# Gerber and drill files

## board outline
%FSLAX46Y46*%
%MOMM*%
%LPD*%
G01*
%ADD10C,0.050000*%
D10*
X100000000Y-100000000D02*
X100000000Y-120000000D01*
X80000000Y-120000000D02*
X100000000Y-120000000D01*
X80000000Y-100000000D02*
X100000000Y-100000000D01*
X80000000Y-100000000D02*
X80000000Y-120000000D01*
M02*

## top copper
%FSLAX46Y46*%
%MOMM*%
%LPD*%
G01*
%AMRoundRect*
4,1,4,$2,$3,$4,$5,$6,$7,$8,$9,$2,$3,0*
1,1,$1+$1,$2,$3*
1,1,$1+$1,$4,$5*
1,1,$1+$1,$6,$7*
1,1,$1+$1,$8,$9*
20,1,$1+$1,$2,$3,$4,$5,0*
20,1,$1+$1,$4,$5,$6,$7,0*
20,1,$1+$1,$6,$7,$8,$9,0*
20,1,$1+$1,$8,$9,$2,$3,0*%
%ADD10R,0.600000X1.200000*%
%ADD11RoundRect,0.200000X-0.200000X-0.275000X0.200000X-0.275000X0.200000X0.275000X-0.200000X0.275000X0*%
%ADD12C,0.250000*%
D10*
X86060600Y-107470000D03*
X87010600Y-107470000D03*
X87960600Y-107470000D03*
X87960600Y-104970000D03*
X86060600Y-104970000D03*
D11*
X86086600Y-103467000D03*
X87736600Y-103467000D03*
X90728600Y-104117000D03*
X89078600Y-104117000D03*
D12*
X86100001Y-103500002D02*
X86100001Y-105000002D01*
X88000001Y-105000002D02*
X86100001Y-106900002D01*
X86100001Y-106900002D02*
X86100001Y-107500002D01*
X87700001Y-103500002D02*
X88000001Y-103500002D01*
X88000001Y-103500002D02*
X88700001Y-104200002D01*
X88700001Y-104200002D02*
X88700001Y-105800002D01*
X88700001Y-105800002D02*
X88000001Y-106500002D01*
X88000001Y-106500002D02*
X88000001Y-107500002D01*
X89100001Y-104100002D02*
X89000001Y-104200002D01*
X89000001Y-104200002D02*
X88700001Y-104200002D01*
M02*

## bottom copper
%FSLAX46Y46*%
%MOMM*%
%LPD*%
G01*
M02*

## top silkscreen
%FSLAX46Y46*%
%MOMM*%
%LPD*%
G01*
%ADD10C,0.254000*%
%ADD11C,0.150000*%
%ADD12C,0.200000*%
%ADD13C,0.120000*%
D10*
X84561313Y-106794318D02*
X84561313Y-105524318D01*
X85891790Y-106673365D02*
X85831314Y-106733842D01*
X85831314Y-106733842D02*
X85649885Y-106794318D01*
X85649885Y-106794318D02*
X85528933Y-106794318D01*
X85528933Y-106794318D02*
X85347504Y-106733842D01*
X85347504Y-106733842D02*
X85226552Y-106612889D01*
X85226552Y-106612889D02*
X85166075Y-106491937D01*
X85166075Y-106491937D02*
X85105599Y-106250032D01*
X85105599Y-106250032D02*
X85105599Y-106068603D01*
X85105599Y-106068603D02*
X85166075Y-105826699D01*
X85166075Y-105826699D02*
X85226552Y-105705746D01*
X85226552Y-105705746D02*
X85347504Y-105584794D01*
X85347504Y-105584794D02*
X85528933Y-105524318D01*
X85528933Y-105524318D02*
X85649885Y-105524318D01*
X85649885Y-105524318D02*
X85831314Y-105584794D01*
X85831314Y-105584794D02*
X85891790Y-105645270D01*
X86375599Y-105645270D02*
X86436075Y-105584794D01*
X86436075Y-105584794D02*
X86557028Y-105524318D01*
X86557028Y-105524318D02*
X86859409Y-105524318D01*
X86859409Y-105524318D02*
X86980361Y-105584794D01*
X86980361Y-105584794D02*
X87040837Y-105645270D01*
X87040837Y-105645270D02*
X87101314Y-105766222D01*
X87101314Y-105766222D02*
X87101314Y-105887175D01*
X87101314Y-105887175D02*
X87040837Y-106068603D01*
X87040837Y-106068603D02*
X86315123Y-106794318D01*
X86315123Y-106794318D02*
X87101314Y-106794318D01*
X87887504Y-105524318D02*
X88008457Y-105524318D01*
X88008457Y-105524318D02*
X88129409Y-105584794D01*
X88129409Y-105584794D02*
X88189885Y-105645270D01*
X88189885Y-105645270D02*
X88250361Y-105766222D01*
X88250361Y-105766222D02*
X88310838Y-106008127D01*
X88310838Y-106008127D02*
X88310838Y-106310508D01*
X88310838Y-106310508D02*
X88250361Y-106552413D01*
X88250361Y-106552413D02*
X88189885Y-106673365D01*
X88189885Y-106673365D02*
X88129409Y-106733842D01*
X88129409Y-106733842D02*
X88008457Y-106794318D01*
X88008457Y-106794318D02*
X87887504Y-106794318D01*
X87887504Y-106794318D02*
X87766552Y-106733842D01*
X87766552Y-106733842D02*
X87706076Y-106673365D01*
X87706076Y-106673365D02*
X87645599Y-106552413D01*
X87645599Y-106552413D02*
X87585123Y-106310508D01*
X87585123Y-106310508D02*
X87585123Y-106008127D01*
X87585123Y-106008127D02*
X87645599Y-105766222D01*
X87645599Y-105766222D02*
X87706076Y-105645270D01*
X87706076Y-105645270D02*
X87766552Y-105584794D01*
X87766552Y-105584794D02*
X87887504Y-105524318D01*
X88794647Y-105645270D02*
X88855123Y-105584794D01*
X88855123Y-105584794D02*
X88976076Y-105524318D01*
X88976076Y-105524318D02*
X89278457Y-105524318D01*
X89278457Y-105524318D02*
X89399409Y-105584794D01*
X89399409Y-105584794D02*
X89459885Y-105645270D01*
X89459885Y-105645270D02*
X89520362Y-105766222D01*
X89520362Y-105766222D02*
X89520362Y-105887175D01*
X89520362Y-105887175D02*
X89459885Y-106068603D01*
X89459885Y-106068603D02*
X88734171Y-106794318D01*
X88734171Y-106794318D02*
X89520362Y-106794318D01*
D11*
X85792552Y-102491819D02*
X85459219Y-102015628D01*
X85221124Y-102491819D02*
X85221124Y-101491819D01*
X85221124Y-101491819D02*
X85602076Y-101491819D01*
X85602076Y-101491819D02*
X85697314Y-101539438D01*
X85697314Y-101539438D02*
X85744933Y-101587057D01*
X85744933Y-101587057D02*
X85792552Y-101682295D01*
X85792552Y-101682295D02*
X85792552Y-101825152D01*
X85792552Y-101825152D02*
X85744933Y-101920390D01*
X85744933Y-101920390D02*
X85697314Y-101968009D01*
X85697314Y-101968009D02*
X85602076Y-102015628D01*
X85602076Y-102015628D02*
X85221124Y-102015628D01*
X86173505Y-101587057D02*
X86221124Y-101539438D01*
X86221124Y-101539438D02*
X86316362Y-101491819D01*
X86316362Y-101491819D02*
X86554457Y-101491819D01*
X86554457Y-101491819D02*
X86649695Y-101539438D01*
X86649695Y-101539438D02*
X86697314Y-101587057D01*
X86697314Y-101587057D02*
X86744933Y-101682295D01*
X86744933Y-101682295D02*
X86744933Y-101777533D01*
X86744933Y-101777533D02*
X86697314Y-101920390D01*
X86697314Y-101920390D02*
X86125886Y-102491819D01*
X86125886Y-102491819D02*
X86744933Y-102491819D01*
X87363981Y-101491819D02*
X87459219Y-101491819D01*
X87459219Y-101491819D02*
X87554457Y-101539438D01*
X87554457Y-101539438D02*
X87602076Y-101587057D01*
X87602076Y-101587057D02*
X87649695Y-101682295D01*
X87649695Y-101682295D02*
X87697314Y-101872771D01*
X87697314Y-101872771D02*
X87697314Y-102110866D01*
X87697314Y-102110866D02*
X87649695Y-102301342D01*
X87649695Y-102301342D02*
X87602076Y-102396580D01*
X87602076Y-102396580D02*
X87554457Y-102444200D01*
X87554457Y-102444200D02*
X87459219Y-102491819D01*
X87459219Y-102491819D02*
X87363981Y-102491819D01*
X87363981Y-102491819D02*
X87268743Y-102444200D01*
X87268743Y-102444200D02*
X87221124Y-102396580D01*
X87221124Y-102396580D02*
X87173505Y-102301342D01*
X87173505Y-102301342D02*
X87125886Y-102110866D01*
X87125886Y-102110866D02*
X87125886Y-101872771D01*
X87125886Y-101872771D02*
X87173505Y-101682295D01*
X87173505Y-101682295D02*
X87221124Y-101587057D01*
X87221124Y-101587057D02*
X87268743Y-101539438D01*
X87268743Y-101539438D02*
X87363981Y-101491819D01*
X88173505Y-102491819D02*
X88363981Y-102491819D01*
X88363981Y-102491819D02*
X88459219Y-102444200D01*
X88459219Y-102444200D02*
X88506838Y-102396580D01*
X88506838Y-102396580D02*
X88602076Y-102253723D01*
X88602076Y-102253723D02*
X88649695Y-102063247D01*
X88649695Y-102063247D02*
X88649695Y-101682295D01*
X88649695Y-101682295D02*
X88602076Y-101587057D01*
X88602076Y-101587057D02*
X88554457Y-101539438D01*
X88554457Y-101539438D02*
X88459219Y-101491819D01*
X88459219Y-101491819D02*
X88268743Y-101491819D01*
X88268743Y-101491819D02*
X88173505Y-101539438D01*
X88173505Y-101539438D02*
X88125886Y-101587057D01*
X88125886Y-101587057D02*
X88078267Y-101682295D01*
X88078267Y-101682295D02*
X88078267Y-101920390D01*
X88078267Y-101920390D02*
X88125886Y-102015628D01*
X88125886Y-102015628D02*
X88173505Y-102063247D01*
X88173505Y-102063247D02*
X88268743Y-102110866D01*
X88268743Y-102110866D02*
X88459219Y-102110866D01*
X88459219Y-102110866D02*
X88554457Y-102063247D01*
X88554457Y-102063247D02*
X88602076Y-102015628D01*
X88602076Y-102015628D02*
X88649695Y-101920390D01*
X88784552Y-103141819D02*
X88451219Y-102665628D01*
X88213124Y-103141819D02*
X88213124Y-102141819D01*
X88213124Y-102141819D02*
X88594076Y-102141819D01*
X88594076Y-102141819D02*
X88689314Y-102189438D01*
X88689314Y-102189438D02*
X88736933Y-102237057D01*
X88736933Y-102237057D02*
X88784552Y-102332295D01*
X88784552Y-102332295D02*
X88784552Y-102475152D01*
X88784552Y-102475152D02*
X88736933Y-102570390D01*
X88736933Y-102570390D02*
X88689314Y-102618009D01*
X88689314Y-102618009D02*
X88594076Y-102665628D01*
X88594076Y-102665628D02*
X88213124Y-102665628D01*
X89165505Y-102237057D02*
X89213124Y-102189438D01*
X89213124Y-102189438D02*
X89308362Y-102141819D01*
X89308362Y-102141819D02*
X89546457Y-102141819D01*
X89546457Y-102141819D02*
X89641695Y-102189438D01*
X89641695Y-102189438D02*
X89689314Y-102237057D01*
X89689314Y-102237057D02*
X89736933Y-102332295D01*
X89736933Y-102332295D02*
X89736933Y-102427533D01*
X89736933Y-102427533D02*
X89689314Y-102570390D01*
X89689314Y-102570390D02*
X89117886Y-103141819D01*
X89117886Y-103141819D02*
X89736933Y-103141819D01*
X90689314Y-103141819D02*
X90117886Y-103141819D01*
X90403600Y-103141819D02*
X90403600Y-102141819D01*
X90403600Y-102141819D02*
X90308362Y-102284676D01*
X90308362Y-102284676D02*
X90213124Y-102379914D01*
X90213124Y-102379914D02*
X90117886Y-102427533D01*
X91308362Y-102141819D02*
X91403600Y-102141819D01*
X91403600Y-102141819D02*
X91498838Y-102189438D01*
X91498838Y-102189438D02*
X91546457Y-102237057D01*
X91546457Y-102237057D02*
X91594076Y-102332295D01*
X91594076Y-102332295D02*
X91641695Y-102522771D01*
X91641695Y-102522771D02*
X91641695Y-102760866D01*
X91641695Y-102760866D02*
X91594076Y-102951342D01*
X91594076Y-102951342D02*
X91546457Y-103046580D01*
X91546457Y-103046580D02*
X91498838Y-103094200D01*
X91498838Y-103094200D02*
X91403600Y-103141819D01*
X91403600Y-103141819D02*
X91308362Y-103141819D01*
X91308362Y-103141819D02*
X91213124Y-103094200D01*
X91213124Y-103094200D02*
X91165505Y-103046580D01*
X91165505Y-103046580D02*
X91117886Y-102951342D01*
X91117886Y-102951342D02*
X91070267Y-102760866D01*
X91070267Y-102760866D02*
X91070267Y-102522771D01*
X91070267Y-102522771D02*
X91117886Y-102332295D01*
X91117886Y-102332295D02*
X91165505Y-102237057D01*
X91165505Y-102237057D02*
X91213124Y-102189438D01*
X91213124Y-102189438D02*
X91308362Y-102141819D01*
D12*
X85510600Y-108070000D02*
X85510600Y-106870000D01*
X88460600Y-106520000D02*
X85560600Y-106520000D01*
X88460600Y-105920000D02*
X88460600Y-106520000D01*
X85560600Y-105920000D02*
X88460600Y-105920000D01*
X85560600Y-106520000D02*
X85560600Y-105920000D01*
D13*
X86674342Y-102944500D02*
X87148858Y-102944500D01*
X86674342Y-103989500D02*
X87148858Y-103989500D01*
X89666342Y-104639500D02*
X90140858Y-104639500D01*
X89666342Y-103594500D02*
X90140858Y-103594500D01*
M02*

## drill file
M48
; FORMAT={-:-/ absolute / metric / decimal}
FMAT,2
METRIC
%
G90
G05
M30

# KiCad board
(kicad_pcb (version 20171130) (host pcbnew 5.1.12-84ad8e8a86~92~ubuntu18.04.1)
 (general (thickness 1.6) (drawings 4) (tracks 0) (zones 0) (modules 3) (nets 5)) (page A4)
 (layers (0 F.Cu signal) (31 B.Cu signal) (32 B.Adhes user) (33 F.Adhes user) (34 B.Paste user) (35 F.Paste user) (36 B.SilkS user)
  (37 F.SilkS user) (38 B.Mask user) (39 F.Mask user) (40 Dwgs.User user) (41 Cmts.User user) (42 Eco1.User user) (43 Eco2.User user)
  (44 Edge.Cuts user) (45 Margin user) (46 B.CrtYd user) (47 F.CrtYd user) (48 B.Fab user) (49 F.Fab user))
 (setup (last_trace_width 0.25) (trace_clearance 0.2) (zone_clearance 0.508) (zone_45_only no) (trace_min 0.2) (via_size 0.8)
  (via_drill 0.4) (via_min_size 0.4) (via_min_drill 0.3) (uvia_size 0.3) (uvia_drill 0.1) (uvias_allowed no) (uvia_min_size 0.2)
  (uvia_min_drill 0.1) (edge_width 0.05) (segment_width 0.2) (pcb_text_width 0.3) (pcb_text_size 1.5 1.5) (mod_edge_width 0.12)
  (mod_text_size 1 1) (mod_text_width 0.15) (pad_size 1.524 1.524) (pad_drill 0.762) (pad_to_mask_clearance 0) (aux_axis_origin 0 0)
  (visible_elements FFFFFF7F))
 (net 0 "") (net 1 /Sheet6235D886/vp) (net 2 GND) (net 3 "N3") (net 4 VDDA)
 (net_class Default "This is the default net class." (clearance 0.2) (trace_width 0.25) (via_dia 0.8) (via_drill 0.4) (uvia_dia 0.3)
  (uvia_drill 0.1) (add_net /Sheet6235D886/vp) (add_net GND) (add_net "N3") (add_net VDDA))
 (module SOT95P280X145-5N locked (layer F.Cu) (at 87.010600 106.220000 90.000000)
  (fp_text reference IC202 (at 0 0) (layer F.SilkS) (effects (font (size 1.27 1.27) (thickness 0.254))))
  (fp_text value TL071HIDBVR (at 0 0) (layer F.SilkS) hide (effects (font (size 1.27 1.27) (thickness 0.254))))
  (fp_line (start -1.85 -1.5) (end -0.65 -1.5) (layer F.SilkS) (width 0.2))
  (fp_line (start -0.3 1.45) (end -0.3 -1.45) (layer F.SilkS) (width 0.2))
  (fp_line (start 0.3 1.45) (end -0.3 1.45) (layer F.SilkS) (width 0.2))
  (fp_line (start 0.3 -1.45) (end 0.3 1.45) (layer F.SilkS) (width 0.2))
  (fp_line (start -0.3 -1.45) (end 0.3 -1.45) (layer F.SilkS) (width 0.2))
  (pad 1 smd rect (at -1.25 -0.95 180.000000) (size 0.6 1.2) (layers F.Cu F.Mask F.Paste) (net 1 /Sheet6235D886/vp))
  (pad 2 smd rect (at -1.25 0 180.000000) (size 0.6 1.2) (layers F.Cu F.Mask F.Paste) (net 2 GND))
  (pad 3 smd rect (at -1.25 0.95 180.000000) (size 0.6 1.2) (layers F.Cu F.Mask F.Paste) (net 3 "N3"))
  (pad 4 smd rect (at 1.25 0.95 180.000000) (size 0.6 1.2) (layers F.Cu F.Mask F.Paste) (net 1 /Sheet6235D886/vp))
  (pad 5 smd rect (at 1.25 -0.95 180.000000) (size 0.6 1.2) (layers F.Cu F.Mask F.Paste) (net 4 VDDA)))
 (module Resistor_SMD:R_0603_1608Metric (layer F.Cu) (at 86.911600 103.467000)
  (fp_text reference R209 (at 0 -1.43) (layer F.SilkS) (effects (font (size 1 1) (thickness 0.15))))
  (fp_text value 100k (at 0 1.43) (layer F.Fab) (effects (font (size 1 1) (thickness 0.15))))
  (fp_line (start -0.237258 -0.5225) (end 0.237258 -0.5225) (layer F.SilkS) (width 0.12))
  (fp_line (start -0.237258 0.5225) (end 0.237258 0.5225) (layer F.SilkS) (width 0.12))
  (pad 1 smd roundrect (at -0.825 0) (size 0.8 0.95) (layers F.Cu F.Mask F.Paste) (roundrect_rratio 0.25) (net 4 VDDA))
  (pad 2 smd roundrect (at 0.825 0) (size 0.8 0.95) (layers F.Cu F.Mask F.Paste) (roundrect_rratio 0.25) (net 3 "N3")))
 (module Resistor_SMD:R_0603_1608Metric (layer F.Cu) (at 89.903600 104.117000)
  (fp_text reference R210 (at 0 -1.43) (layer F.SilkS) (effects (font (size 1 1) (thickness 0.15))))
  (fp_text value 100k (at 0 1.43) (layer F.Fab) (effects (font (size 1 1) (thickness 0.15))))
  (fp_line (start -0.237258 0.5225) (end 0.237258 0.5225) (layer F.SilkS) (width 0.12))
  (fp_line (start -0.237258 -0.5225) (end 0.237258 -0.5225) (layer F.SilkS) (width 0.12))
  (pad 2 smd roundrect (at 0.825 0) (size 0.8 0.95) (layers F.Cu F.Mask F.Paste) (roundrect_rratio 0.25) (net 2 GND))
  (pad 1 smd roundrect (at -0.825 0) (size 0.8 0.95) (layers F.Cu F.Mask F.Paste) (roundrect_rratio 0.25) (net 3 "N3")))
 (gr_line (start 100 100) (end 100 120) (layer Edge.Cuts) (width 0.05))
 (gr_line (start 80 120) (end 100 120) (layer Edge.Cuts) (width 0.05))
 (gr_line (start 80 100) (end 100 100) (layer Edge.Cuts) (width 0.05))
 (gr_line (start 80 100) (end 80 120) (layer Edge.Cuts) (width 0.05))
 (segment (start 86.100001 103.500002) (end 86.100001 105.000002) (width 0.250000) (layer F.Cu) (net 4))
 (segment (start 88.000001 105.000002) (end 86.100001 106.900002) (width 0.250000) (layer F.Cu) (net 1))
 (segment (start 86.100001 106.900002) (end 86.100001 107.500002) (width 0.250000) (layer F.Cu) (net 1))
 (segment (start 87.700001 103.500002) (end 88.000001 103.500002) (width 0.250000) (layer F.Cu) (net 3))
 (segment (start 88.000001 103.500002) (end 88.700001 104.200002) (width 0.250000) (layer F.Cu) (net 3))
 (segment (start 88.700001 104.200002) (end 88.700001 105.800002) (width 0.250000) (layer F.Cu) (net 3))
 (segment (start 88.700001 105.800002) (end 88.000001 106.500002) (width 0.250000) (layer F.Cu) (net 3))
 (segment (start 88.000001 106.500002) (end 88.000001 107.500002) (width 0.250000) (layer F.Cu) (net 3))
 (segment (start 89.100001 104.100002) (end 89.000001 104.200002) (width 0.250000) (layer F.Cu) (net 3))
 (segment (start 89.000001 104.200002) (end 88.700001 104.200002) (width 0.250000) (layer F.Cu) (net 3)))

